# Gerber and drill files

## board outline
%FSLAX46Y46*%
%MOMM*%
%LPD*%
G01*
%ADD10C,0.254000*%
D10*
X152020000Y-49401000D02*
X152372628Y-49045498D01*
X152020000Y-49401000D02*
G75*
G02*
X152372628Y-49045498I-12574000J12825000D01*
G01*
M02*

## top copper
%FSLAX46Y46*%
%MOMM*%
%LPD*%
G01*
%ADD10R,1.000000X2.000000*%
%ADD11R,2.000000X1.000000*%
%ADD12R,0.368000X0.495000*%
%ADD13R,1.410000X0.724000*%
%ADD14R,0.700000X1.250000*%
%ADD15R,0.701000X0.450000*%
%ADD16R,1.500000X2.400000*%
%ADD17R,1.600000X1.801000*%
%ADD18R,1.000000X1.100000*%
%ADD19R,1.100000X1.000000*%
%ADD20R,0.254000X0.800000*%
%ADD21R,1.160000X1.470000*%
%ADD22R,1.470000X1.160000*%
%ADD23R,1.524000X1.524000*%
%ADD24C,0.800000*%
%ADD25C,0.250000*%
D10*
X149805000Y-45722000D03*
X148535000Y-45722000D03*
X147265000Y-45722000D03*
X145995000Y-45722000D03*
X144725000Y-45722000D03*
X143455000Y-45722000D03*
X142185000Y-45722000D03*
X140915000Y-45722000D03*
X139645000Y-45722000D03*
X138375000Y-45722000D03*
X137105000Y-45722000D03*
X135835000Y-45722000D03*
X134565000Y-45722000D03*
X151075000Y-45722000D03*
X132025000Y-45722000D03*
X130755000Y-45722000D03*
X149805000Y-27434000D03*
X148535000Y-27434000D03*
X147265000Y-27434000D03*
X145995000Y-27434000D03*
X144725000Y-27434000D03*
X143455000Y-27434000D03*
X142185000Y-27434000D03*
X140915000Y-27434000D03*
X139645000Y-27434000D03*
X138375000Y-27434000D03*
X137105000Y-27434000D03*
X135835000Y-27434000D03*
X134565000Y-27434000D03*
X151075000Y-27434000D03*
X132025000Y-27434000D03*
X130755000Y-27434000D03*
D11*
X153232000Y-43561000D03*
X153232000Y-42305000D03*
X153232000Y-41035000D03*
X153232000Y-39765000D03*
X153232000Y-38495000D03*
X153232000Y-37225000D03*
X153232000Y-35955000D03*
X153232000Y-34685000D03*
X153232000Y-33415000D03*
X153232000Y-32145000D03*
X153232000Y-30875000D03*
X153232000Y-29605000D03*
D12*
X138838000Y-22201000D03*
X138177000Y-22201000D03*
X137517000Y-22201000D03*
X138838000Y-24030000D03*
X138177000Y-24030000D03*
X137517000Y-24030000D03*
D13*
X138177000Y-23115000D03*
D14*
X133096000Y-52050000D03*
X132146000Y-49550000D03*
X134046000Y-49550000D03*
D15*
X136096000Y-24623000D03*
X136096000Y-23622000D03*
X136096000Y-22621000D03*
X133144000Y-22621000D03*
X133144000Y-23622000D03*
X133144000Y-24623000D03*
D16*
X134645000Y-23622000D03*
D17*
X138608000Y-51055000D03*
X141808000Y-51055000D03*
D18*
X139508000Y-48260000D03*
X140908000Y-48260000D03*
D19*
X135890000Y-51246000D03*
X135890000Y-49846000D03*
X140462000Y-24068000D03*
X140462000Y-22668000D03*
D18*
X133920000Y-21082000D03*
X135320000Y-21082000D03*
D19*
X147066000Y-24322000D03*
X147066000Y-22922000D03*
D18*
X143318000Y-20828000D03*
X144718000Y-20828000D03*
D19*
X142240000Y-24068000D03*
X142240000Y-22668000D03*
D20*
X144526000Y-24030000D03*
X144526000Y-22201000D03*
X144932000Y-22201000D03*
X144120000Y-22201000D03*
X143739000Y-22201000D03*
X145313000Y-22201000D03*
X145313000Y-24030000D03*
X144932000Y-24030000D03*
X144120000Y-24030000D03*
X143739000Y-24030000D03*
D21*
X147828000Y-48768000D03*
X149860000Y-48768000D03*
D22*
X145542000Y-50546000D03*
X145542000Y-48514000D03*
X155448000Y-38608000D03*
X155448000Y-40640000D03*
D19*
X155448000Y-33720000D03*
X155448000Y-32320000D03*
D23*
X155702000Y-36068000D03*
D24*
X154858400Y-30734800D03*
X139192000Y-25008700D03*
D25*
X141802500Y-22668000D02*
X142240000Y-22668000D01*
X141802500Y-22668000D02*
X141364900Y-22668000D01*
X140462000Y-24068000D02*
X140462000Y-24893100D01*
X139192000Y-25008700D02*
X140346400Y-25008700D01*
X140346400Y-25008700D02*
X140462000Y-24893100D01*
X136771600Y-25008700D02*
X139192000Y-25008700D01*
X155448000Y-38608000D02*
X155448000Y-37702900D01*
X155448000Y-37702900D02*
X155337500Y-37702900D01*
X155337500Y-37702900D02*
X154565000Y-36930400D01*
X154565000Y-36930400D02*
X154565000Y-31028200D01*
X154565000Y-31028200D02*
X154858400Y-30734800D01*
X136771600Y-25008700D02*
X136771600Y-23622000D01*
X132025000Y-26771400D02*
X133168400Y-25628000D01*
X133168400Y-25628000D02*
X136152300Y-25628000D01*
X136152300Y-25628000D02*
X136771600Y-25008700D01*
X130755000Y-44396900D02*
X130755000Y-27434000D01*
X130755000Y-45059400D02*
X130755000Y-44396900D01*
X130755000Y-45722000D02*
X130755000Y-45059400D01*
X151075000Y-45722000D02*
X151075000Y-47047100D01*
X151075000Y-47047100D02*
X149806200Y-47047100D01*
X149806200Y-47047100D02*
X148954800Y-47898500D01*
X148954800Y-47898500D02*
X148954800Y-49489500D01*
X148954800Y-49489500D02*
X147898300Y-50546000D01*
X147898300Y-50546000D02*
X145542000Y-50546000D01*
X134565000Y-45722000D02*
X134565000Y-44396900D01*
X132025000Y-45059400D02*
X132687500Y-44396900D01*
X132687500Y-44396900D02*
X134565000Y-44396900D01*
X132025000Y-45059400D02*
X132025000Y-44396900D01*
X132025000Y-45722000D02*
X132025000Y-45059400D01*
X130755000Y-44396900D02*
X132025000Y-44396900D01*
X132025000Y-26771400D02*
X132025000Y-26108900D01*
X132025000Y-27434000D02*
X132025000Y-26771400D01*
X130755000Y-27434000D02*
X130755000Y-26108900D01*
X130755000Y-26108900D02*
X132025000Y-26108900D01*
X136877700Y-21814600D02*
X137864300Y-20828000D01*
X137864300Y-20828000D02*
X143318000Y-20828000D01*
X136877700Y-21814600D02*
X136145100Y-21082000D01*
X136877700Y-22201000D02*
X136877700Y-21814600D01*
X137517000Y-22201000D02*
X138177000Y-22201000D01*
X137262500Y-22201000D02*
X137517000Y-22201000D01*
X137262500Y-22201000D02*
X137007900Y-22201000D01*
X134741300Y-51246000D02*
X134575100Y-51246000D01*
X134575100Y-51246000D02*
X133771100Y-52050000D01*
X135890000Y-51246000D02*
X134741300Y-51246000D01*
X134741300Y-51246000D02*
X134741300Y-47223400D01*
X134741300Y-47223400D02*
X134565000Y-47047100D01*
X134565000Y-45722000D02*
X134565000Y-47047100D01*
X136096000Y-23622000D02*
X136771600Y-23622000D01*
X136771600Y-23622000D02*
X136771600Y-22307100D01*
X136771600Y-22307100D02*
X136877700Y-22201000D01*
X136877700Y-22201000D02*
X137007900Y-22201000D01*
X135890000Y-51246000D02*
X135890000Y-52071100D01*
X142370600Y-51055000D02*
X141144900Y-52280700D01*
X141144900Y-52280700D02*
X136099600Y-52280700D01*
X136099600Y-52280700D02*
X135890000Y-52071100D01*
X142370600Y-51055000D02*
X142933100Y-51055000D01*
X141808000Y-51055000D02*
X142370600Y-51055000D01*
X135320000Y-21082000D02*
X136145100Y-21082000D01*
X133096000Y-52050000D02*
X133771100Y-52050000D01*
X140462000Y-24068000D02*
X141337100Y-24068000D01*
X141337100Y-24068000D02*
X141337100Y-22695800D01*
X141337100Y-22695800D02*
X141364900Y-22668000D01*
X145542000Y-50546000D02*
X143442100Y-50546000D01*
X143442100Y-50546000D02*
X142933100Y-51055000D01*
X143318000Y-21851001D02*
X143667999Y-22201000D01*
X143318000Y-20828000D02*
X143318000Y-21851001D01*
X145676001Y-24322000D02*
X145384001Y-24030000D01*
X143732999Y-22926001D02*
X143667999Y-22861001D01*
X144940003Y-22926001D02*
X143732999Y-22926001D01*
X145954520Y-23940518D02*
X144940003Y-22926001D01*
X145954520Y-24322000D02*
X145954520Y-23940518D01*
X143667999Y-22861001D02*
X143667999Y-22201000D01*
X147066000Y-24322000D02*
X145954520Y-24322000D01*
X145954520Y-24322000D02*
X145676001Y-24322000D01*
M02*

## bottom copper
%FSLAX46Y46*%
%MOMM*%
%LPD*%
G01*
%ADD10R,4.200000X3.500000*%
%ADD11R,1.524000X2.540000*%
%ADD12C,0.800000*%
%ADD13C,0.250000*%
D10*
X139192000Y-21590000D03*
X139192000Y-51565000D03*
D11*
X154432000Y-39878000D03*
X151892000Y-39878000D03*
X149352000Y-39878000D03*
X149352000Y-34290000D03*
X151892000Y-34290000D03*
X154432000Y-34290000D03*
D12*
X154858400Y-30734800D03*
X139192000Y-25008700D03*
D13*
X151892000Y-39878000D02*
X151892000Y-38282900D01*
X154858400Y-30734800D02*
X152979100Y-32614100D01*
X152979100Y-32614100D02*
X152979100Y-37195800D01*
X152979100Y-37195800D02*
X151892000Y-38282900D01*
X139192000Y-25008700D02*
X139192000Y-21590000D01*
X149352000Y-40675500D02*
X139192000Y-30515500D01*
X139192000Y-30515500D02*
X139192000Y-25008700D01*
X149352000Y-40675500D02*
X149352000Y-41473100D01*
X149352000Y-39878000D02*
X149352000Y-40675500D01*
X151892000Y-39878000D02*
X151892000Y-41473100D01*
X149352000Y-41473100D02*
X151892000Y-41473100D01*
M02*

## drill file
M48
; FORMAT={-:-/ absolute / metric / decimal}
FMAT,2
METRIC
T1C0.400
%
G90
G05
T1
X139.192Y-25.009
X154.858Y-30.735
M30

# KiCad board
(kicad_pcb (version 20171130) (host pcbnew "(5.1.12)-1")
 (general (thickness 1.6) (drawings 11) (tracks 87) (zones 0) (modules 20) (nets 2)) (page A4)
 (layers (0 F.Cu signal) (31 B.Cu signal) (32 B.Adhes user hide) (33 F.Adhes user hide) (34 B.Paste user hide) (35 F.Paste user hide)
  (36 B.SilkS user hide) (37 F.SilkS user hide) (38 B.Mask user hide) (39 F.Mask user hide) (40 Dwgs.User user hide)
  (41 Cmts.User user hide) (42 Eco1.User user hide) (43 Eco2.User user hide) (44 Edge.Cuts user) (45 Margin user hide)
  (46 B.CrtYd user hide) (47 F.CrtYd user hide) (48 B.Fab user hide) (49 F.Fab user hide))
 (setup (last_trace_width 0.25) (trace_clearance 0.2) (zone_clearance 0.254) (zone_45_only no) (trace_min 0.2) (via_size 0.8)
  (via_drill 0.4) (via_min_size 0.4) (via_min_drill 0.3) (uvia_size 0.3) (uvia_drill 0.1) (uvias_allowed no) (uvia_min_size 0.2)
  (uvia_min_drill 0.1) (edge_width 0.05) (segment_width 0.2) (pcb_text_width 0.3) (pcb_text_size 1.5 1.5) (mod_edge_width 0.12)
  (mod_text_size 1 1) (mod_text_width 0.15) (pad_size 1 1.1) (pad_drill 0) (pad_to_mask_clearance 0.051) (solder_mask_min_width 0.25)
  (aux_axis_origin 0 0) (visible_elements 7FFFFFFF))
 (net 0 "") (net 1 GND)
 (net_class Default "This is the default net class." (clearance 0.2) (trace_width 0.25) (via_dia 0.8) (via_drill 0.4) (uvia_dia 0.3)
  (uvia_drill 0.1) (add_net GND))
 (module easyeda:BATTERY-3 (layer F.Cu) (at 139.192 36.577)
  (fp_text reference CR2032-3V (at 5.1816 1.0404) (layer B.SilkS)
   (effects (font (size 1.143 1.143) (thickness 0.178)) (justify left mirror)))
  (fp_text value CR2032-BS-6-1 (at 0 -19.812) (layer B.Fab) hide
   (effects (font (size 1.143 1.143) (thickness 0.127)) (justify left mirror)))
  (pad 2 smd rect (at 0 -14.987 270) (size 3.5 4.2) (layers B.Cu B.Paste B.Mask) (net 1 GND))
  (pad 1 smd rect (at 0 14.988 270) (size 3.5 4.2) (layers B.Cu B.Paste B.Mask)))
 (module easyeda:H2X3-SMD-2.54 (layer F.Cu) (at 151.892 37.084 270)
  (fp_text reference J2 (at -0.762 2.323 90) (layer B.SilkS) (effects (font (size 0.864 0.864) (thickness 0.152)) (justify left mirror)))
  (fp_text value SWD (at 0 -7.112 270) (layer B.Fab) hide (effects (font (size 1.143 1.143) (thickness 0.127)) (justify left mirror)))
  (pad 1 smd rect (at 2.794 -2.54 270) (size 2.54 1.524) (layers B.Cu B.Paste B.Mask))
  (pad 2 smd rect (at 2.794 0 270) (size 2.54 1.524) (layers B.Cu B.Paste B.Mask) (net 1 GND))
  (pad 3 smd rect (at 2.794 2.54 270) (size 2.54 1.524) (layers B.Cu B.Paste B.Mask) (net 1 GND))
  (pad 4 smd rect (at -2.794 2.54 90) (size 2.54 1.524) (layers B.Cu B.Paste B.Mask))
  (pad 5 smd rect (at -2.794 0 90) (size 2.54 1.524) (layers B.Cu B.Paste B.Mask))
  (pad 6 smd rect (at -2.794 -2.54 90) (size 2.54 1.524) (layers B.Cu B.Paste B.Mask)))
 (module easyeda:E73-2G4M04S (layer F.Cu) (at 129.358 45.34 90)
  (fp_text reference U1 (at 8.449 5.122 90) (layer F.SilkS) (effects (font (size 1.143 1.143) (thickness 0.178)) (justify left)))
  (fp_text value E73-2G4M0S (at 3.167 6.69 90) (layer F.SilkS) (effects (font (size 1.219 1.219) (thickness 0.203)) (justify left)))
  (pad 14 smd rect (at -0.382 20.447 90) (size 2 1) (layers F.Cu F.Paste F.Mask))
  (pad 13 smd rect (at -0.382 19.177 90) (size 2 1) (layers F.Cu F.Paste F.Mask))
  (pad 12 smd rect (at -0.382 17.907 90) (size 2 1) (layers F.Cu F.Paste F.Mask))
  (pad 11 smd rect (at -0.382 16.637 90) (size 2 1) (layers F.Cu F.Paste F.Mask))
  (pad 10 smd rect (at -0.382 15.367 90) (size 2 1) (layers F.Cu F.Paste F.Mask))
  (pad 9 smd rect (at -0.382 14.097 90) (size 2 1) (layers F.Cu F.Paste F.Mask))
  (pad 8 smd rect (at -0.382 12.827 90) (size 2 1) (layers F.Cu F.Paste F.Mask))
  (pad 7 smd rect (at -0.382 11.557 90) (size 2 1) (layers F.Cu F.Paste F.Mask))
  (pad 6 smd rect (at -0.382 10.287 90) (size 2 1) (layers F.Cu F.Paste F.Mask))
  (pad 5 smd rect (at -0.382 9.017 90) (size 2 1) (layers F.Cu F.Paste F.Mask))
  (pad 4 smd rect (at -0.382 7.747 90) (size 2 1) (layers F.Cu F.Paste F.Mask))
  (pad 3 smd rect (at -0.382 6.477 90) (size 2 1) (layers F.Cu F.Paste F.Mask))
  (pad 2 smd rect (at -0.382 5.207 90) (size 2 1) (layers F.Cu F.Paste F.Mask) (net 1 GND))
  (pad 15 smd rect (at -0.382 21.717 90) (size 2 1) (layers F.Cu F.Paste F.Mask) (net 1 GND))
  (pad 1 smd rect (at -0.382 2.667 90) (size 2 1) (layers F.Cu F.Paste F.Mask) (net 1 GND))
  (pad 0 smd rect (at -0.382 1.397 90) (size 2 1) (layers F.Cu F.Paste F.Mask) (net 1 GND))
  (pad 29 smd rect (at 17.906 20.447 90) (size 2 1) (layers F.Cu F.Paste F.Mask))
  (pad 30 smd rect (at 17.906 19.177 90) (size 2 1) (layers F.Cu F.Paste F.Mask))
  (pad 31 smd rect (at 17.906 17.907 90) (size 2 1) (layers F.Cu F.Paste F.Mask))
  (pad 32 smd rect (at 17.906 16.637 90) (size 2 1) (layers F.Cu F.Paste F.Mask))
  (pad 33 smd rect (at 17.906 15.367 90) (size 2 1) (layers F.Cu F.Paste F.Mask))
  (pad 34 smd rect (at 17.906 14.097 90) (size 2 1) (layers F.Cu F.Paste F.Mask))
  (pad 35 smd rect (at 17.906 12.827 90) (size 2 1) (layers F.Cu F.Paste F.Mask))
  (pad 36 smd rect (at 17.906 11.557 90) (size 2 1) (layers F.Cu F.Paste F.Mask))
  (pad 37 smd rect (at 17.906 10.287 90) (size 2 1) (layers F.Cu F.Paste F.Mask))
  (pad 38 smd rect (at 17.906 9.017 90) (size 2 1) (layers F.Cu F.Paste F.Mask))
  (pad 39 smd rect (at 17.906 7.747 90) (size 2 1) (layers F.Cu F.Paste F.Mask))
  (pad 40 smd rect (at 17.906 6.477 90) (size 2 1) (layers F.Cu F.Paste F.Mask))
  (pad 41 smd rect (at 17.906 5.207 90) (size 2 1) (layers F.Cu F.Paste F.Mask))
  (pad 28 smd rect (at 17.906 21.717 90) (size 2 1) (layers F.Cu F.Paste F.Mask))
  (pad 42 smd rect (at 17.906 2.667 90) (size 2 1) (layers F.Cu F.Paste F.Mask) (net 1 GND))
  (pad 43 smd rect (at 17.906 1.397 90) (size 2 1) (layers F.Cu F.Paste F.Mask) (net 1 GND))
  (pad 16 smd rect (at 1.779 23.874 180) (size 2 1) (layers F.Cu F.Paste F.Mask))
  (pad 17 smd rect (at 3.035 23.874 180) (size 2 1) (layers F.Cu F.Paste F.Mask))
  (pad 18 smd rect (at 4.305 23.874 180) (size 2 1) (layers F.Cu F.Paste F.Mask))
  (pad 19 smd rect (at 5.575 23.874 180) (size 2 1) (layers F.Cu F.Paste F.Mask))
  (pad 20 smd rect (at 6.845 23.874 180) (size 2 1) (layers F.Cu F.Paste F.Mask))
  (pad 21 smd rect (at 8.115 23.874 180) (size 2 1) (layers F.Cu F.Paste F.Mask))
  (pad 22 smd rect (at 9.385 23.874 180) (size 2 1) (layers F.Cu F.Paste F.Mask))
  (pad 23 smd rect (at 10.655 23.874 180) (size 2 1) (layers F.Cu F.Paste F.Mask))
  (pad 24 smd rect (at 11.925 23.874 180) (size 2 1) (layers F.Cu F.Paste F.Mask))
  (pad 25 smd rect (at 13.195 23.874 180) (size 2 1) (layers F.Cu F.Paste F.Mask))
  (pad 26 smd rect (at 14.465 23.874 180) (size 2 1) (layers F.Cu F.Paste F.Mask))
  (pad 27 smd rect (at 15.735 23.874 180) (size 2 1) (layers F.Cu F.Paste F.Mask)))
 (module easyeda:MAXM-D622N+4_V (layer F.Cu) (at 138.176 23.114 270)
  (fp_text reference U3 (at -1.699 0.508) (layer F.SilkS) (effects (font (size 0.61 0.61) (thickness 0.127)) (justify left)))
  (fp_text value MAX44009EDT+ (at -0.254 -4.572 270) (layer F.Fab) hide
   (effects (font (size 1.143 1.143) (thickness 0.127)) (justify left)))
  (pad 1 smd rect (at -0.913 -0.662) (size 0.368 0.495) (layers F.Cu F.Paste F.Mask))
  (pad 2 smd rect (at -0.913 -0.001) (size 0.368 0.495) (layers F.Cu F.Paste F.Mask) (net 1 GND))
  (pad 3 smd rect (at -0.913 0.659) (size 0.368 0.495) (layers F.Cu F.Paste F.Mask) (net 1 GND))
  (pad 6 smd rect (at 0.916 -0.662) (size 0.368 0.495) (layers F.Cu F.Paste F.Mask))
  (pad 5 smd rect (at 0.916 -0.001) (size 0.368 0.495) (layers F.Cu F.Paste F.Mask))
  (pad 4 smd rect (at 0.916 0.659) (size 0.368 0.495) (layers F.Cu F.Paste F.Mask))
  (pad 7 smd rect (at 0.001 -0.001) (size 1.41 0.724) (layers F.Cu F.Paste F.Mask)))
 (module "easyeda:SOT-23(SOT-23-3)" (layer F.Cu) (at 133.096 50.8 180)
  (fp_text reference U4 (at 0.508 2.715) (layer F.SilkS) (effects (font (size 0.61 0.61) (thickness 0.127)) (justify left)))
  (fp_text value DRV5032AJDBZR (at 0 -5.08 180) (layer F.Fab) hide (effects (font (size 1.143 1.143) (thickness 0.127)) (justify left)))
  (pad 3 smd rect (at 0 -1.25) (size 0.7 1.25) (layers F.Cu F.Paste F.Mask) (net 1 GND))
  (pad 2 smd rect (at 0.95 1.25) (size 0.7 1.25) (layers F.Cu F.Paste F.Mask))
  (pad 1 smd rect (at -0.95 1.25) (size 0.7 1.25) (layers F.Cu F.Paste F.Mask)))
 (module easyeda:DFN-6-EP (layer F.Cu) (at 134.62 23.622 90)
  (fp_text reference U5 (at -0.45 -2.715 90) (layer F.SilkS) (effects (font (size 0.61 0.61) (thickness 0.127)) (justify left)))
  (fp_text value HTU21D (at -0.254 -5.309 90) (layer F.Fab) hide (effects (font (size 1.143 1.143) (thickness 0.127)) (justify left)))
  (pad 1 smd rect (at -1.001 1.476 90) (size 0.45 0.701) (layers F.Cu F.Paste F.Mask))
  (pad 2 smd rect (at 0 1.476 90) (size 0.45 0.701) (layers F.Cu F.Paste F.Mask) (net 1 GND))
  (pad 3 smd rect (at 1.001 1.476 90) (size 0.45 0.701) (layers F.Cu F.Paste F.Mask))
  (pad 4 smd rect (at 1.001 -1.476 90) (size 0.45 0.701) (layers F.Cu F.Paste F.Mask))
  (pad 5 smd rect (at 0 -1.476 90) (size 0.45 0.701) (layers F.Cu F.Paste F.Mask))
  (pad 6 smd rect (at -1.001 -1.476 90) (size 0.45 0.701) (layers F.Cu F.Paste F.Mask))
  (pad 7 smd rect (at 0 0.025 90) (size 2.4 1.5) (layers F.Cu F.Paste F.Mask)))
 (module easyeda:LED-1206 (layer F.Cu) (at 140.208 51.054 180)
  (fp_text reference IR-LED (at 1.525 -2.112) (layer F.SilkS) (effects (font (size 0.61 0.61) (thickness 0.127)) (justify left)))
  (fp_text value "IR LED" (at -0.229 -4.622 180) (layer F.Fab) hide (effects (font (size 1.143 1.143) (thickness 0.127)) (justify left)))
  (pad 1 smd rect (at 1.6 -0.001) (size 1.6 1.801) (layers F.Cu F.Paste F.Mask))
  (pad 2 smd rect (at -1.6 -0.001) (size 1.6 1.801) (layers F.Cu F.Paste F.Mask) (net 1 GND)))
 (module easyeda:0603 (layer F.Cu) (at 140.208 48.26)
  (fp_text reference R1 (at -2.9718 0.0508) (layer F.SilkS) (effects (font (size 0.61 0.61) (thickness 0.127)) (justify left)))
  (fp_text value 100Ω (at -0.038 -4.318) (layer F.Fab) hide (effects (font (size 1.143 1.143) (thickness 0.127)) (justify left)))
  (pad 1 smd rect (at -0.7 0) (size 1 1.1) (layers F.Cu F.Paste F.Mask))
  (pad 2 smd rect (at 0.7 0) (size 1 1.1) (layers F.Cu F.Paste F.Mask)))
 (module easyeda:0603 (layer F.Cu) (at 135.89 50.546 90)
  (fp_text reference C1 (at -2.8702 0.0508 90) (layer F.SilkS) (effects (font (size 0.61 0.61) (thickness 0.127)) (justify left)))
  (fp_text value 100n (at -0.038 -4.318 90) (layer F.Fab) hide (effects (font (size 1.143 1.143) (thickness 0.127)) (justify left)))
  (pad 1 smd rect (at -0.7 0 90) (size 1 1.1) (layers F.Cu F.Paste F.Mask) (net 1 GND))
  (pad 2 smd rect (at 0.7 0 90) (size 1 1.1) (layers F.Cu F.Paste F.Mask)))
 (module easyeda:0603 (layer F.Cu) (at 140.462 23.368 90)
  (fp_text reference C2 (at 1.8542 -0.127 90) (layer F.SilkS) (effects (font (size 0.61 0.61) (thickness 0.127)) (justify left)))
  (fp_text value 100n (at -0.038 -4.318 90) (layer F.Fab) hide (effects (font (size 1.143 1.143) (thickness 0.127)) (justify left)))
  (pad 1 smd rect (at -0.7 0 90) (size 1 1.1) (layers F.Cu F.Paste F.Mask) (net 1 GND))
  (pad 2 smd rect (at 0.7 0 90) (size 1 1.1) (layers F.Cu F.Paste F.Mask)))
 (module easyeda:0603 (layer F.Cu) (at 134.62 21.082)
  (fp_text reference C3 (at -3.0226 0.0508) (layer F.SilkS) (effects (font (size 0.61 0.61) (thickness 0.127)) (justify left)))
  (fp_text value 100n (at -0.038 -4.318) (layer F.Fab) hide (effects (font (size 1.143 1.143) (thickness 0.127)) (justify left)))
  (pad 1 smd rect (at -0.7 0) (size 1 1.1) (layers F.Cu F.Paste F.Mask))
  (pad 2 smd rect (at 0.7 0) (size 1 1.1) (layers F.Cu F.Paste F.Mask) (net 1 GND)))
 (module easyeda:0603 (layer F.Cu) (at 147.066 23.622 90)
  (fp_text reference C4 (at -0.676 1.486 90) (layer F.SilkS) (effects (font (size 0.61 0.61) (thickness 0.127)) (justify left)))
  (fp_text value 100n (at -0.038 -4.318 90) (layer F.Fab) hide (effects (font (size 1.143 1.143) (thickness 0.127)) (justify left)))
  (pad 1 smd rect (at -0.7 0 90) (size 1 1.1) (layers F.Cu F.Paste F.Mask) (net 1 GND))
  (pad 2 smd rect (at 0.7 0 90) (size 1 1.1) (layers F.Cu F.Paste F.Mask)))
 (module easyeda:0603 (layer F.Cu) (at 144.018 20.828)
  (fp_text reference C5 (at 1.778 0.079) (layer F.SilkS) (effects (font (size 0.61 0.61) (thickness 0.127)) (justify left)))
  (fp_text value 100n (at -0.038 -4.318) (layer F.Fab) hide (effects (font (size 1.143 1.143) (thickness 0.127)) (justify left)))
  (pad 1 smd rect (at -0.7 0) (size 1 1.1) (layers F.Cu F.Paste F.Mask) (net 1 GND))
  (pad 2 smd rect (at 0.7 0) (size 1 1.1) (layers F.Cu F.Paste F.Mask)))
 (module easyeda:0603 (layer F.Cu) (at 142.24 23.368 90)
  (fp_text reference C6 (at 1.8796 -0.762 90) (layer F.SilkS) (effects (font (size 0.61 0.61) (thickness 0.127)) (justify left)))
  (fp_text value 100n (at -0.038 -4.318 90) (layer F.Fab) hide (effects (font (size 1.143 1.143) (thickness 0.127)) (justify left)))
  (pad 1 smd rect (at -0.7 0 90) (size 1 1.1) (layers F.Cu F.Paste F.Mask))
  (pad 2 smd rect (at 0.7 0 90) (size 1 1.1) (layers F.Cu F.Paste F.Mask) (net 1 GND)))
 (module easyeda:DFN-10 (layer F.Cu) (at 144.526 23.114 270)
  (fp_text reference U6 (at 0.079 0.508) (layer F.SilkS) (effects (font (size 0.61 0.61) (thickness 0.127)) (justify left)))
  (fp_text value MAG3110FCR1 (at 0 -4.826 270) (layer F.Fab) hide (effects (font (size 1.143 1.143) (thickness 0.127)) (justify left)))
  (pad 8 smd rect (at 0.916 0 270) (size 0.8 0.254) (layers F.Cu F.Paste F.Mask))
  (pad 3 smd rect (at -0.913 0 270) (size 0.8 0.254) (layers F.Cu F.Paste F.Mask))
  (pad 2 smd rect (at -0.913 -0.406 270) (size 0.8 0.254) (layers F.Cu F.Paste F.Mask))
  (pad 4 smd rect (at -0.913 0.406 270) (size 0.8 0.254) (layers F.Cu F.Paste F.Mask))
  (pad 5 smd rect (at -0.913 0.787 270) (size 0.8 0.254) (layers F.Cu F.Paste F.Mask) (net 1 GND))
  (pad 1 smd rect (at -0.913 -0.787 270) (size 0.8 0.254) (layers F.Cu F.Paste F.Mask))
  (pad 10 smd rect (at 0.916 -0.787 270) (size 0.8 0.254) (layers F.Cu F.Paste F.Mask) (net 1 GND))
  (pad 9 smd rect (at 0.916 -0.406 270) (size 0.8 0.254) (layers F.Cu F.Paste F.Mask))
  (pad 7 smd rect (at 0.916 0.406 270) (size 0.8 0.254) (layers F.Cu F.Paste F.Mask))
  (pad 6 smd rect (at 0.916 0.787 270) (size 0.8 0.254) (layers F.Cu F.Paste F.Mask)))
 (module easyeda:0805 (layer F.Cu) (at 147.828 48.768)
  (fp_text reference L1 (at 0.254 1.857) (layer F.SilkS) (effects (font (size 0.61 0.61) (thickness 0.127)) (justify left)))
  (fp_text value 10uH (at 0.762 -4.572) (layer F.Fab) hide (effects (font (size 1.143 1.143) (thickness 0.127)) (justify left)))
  (pad 1 smd rect (at 0 0) (size 1.16 1.47) (layers F.Cu F.Paste F.Mask))
  (pad 2 smd rect (at 2.032 0) (size 1.16 1.47) (layers F.Cu F.Paste F.Mask)))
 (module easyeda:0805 (layer F.Cu) (at 145.542 50.546 90)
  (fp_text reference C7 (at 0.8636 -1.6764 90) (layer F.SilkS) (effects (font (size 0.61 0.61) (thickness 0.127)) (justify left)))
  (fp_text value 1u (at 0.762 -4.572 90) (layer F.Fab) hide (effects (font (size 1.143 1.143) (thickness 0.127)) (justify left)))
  (pad 1 smd rect (at 0 0 90) (size 1.16 1.47) (layers F.Cu F.Paste F.Mask) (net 1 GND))
  (pad 2 smd rect (at 2.032 0 90) (size 1.16 1.47) (layers F.Cu F.Paste F.Mask)))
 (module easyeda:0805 (layer F.Cu) (at 155.448 38.608 270)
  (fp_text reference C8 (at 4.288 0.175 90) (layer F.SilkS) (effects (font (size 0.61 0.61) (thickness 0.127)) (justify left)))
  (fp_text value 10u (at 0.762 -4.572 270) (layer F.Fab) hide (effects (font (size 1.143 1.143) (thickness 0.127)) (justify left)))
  (pad 1 smd rect (at 0 0 270) (size 1.16 1.47) (layers F.Cu F.Paste F.Mask) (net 1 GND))
  (pad 2 smd rect (at 2.032 0 270) (size 1.16 1.47) (layers F.Cu F.Paste F.Mask)))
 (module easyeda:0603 (layer F.Cu) (at 155.448 33.02 90)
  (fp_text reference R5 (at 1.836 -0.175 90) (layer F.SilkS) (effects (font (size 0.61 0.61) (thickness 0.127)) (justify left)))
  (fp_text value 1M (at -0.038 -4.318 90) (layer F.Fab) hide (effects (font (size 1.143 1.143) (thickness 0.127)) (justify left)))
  (pad 1 smd rect (at -0.7 0 90) (size 1 1.1) (layers F.Cu F.Paste F.Mask))
  (pad 2 smd rect (at 0.7 0 90) (size 1 1.1) (layers F.Cu F.Paste F.Mask)))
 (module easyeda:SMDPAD (layer F.Cu) (at 155.702 36.068)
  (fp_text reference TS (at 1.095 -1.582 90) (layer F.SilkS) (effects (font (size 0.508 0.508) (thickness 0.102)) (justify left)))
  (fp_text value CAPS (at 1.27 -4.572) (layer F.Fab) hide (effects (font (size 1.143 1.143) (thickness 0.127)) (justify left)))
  (pad 1 smd rect (at 0 0) (size 1.524 1.524) (layers F.Cu F.Paste F.Mask)))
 (gr_line (start 152.02 49.401) (end 152.372628 49.045498) (layer Edge.Cuts) (width 0.254))
 (gr_arc (start 139.446 36.576) (end 152.02 49.401) (angle 358.4025929) (layer Edge.Cuts) (width 0.254))
 (segment (start 141.8025 22.668) (end 142.24 22.668) (width 0.25) (layer F.Cu) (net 1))
 (segment (start 141.8025 22.668) (end 141.3649 22.668) (width 0.25) (layer F.Cu) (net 1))
 (segment (start 140.462 24.068) (end 140.462 24.8931) (width 0.25) (layer F.Cu) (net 1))
 (segment (start 139.192 25.0087) (end 140.3464 25.0087) (width 0.25) (layer F.Cu) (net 1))
 (segment (start 140.3464 25.0087) (end 140.462 24.8931) (width 0.25) (layer F.Cu) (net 1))
 (segment (start 136.7716 25.0087) (end 139.192 25.0087) (width 0.25) (layer F.Cu) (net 1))
 (segment (start 155.448 38.608) (end 155.448 37.7029) (width 0.25) (layer F.Cu) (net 1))
 (segment (start 151.892 39.878) (end 151.892 38.2829) (width 0.25) (layer B.Cu) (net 1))
 (segment (start 155.448 37.7029) (end 155.3375 37.7029) (width 0.25) (layer F.Cu) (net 1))
 (segment (start 155.3375 37.7029) (end 154.565 36.9304) (width 0.25) (layer F.Cu) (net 1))
 (segment (start 154.565 36.9304) (end 154.565 31.0282) (width 0.25) (layer F.Cu) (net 1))
 (segment (start 154.565 31.0282) (end 154.8584 30.7348) (width 0.25) (layer F.Cu) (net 1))
 (segment (start 154.8584 30.7348) (end 152.9791 32.6141) (width 0.25) (layer B.Cu) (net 1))
 (segment (start 152.9791 32.6141) (end 152.9791 37.1958) (width 0.25) (layer B.Cu) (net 1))
 (segment (start 152.9791 37.1958) (end 151.892 38.2829) (width 0.25) (layer B.Cu) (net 1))
 (segment (start 139.192 25.0087) (end 139.192 21.59) (width 0.25) (layer B.Cu) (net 1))
 (segment (start 149.352 40.6755) (end 139.192 30.5155) (width 0.25) (layer B.Cu) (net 1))
 (segment (start 139.192 30.5155) (end 139.192 25.0087) (width 0.25) (layer B.Cu) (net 1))
 (segment (start 136.7716 25.0087) (end 136.7716 23.622) (width 0.25) (layer F.Cu) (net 1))
 (segment (start 132.025 26.7714) (end 133.1684 25.628) (width 0.25) (layer F.Cu) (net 1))
 (segment (start 133.1684 25.628) (end 136.1523 25.628) (width 0.25) (layer F.Cu) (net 1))
 (segment (start 136.1523 25.628) (end 136.7716 25.0087) (width 0.25) (layer F.Cu) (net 1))
 (segment (start 149.352 40.6755) (end 149.352 41.4731) (width 0.25) (layer B.Cu) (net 1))
 (segment (start 149.352 39.878) (end 149.352 40.6755) (width 0.25) (layer B.Cu) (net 1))
 (segment (start 151.892 39.878) (end 151.892 41.4731) (width 0.25) (layer B.Cu) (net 1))
 (segment (start 149.352 41.4731) (end 151.892 41.4731) (width 0.25) (layer B.Cu) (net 1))
 (segment (start 130.755 44.3969) (end 130.755 27.434) (width 0.25) (layer F.Cu) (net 1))
 (segment (start 130.755 45.0594) (end 130.755 44.3969) (width 0.25) (layer F.Cu) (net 1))
 (segment (start 130.755 45.722) (end 130.755 45.0594) (width 0.25) (layer F.Cu) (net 1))
 (segment (start 151.075 45.722) (end 151.075 47.0471) (width 0.25) (layer F.Cu) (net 1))
 (segment (start 151.075 47.0471) (end 149.8062 47.0471) (width 0.25) (layer F.Cu) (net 1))
 (segment (start 149.8062 47.0471) (end 148.9548 47.8985) (width 0.25) (layer F.Cu) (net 1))
 (segment (start 148.9548 47.8985) (end 148.9548 49.4895) (width 0.25) (layer F.Cu) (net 1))
 (segment (start 148.9548 49.4895) (end 147.8983 50.546) (width 0.25) (layer F.Cu) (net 1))
 (segment (start 147.8983 50.546) (end 145.542 50.546) (width 0.25) (layer F.Cu) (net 1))
 (segment (start 134.565 45.722) (end 134.565 44.3969) (width 0.25) (layer F.Cu) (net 1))
 (segment (start 132.025 45.0594) (end 132.6875 44.3969) (width 0.25) (layer F.Cu) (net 1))
 (segment (start 132.6875 44.3969) (end 134.565 44.3969) (width 0.25) (layer F.Cu) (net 1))
 (segment (start 132.025 45.0594) (end 132.025 44.3969) (width 0.25) (layer F.Cu) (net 1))
 (segment (start 132.025 45.722) (end 132.025 45.0594) (width 0.25) (layer F.Cu) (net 1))
 (segment (start 130.755 44.3969) (end 132.025 44.3969) (width 0.25) (layer F.Cu) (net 1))
 (segment (start 132.025 26.7714) (end 132.025 26.1089) (width 0.25) (layer F.Cu) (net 1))
 (segment (start 132.025 27.434) (end 132.025 26.7714) (width 0.25) (layer F.Cu) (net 1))
 (segment (start 130.755 27.434) (end 130.755 26.1089) (width 0.25) (layer F.Cu) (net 1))
 (segment (start 130.755 26.1089) (end 132.025 26.1089) (width 0.25) (layer F.Cu) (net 1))
 (segment (start 136.8777 21.8146) (end 137.8643 20.828) (width 0.25) (layer F.Cu) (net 1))
 (segment (start 137.8643 20.828) (end 143.318 20.828) (width 0.25) (layer F.Cu) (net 1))
 (segment (start 136.8777 21.8146) (end 136.1451 21.082) (width 0.25) (layer F.Cu) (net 1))
 (segment (start 136.8777 22.201) (end 136.8777 21.8146) (width 0.25) (layer F.Cu) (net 1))
 (segment (start 137.517 22.201) (end 138.177 22.201) (width 0.25) (layer F.Cu) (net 1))
 (segment (start 137.2625 22.201) (end 137.517 22.201) (width 0.25) (layer F.Cu) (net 1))
 (segment (start 137.2625 22.201) (end 137.0079 22.201) (width 0.25) (layer F.Cu) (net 1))
 (segment (start 134.7413 51.246) (end 134.5751 51.246) (width 0.25) (layer F.Cu) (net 1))
 (segment (start 134.5751 51.246) (end 133.7711 52.05) (width 0.25) (layer F.Cu) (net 1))
 (segment (start 135.89 51.246) (end 134.7413 51.246) (width 0.25) (layer F.Cu) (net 1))
 (segment (start 134.7413 51.246) (end 134.7413 47.2234) (width 0.25) (layer F.Cu) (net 1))
 (segment (start 134.7413 47.2234) (end 134.565 47.0471) (width 0.25) (layer F.Cu) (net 1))
 (segment (start 134.565 45.722) (end 134.565 47.0471) (width 0.25) (layer F.Cu) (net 1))
 (segment (start 136.096 23.622) (end 136.7716 23.622) (width 0.25) (layer F.Cu) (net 1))
 (segment (start 136.7716 23.622) (end 136.7716 22.3071) (width 0.25) (layer F.Cu) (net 1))
 (segment (start 136.7716 22.3071) (end 136.8777 22.201) (width 0.25) (layer F.Cu) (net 1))
 (segment (start 136.8777 22.201) (end 137.0079 22.201) (width 0.25) (layer F.Cu) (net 1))
 (segment (start 135.89 51.246) (end 135.89 52.0711) (width 0.25) (layer F.Cu) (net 1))
 (segment (start 142.3706 51.055) (end 141.1449 52.2807) (width 0.25) (layer F.Cu) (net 1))
 (segment (start 141.1449 52.2807) (end 136.0996 52.2807) (width 0.25) (layer F.Cu) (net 1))
 (segment (start 136.0996 52.2807) (end 135.89 52.0711) (width 0.25) (layer F.Cu) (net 1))
 (segment (start 142.3706 51.055) (end 142.9331 51.055) (width 0.25) (layer F.Cu) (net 1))
 (segment (start 141.808 51.055) (end 142.3706 51.055) (width 0.25) (layer F.Cu) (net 1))
 (segment (start 135.32 21.082) (end 136.1451 21.082) (width 0.25) (layer F.Cu) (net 1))
 (segment (start 133.096 52.05) (end 133.7711 52.05) (width 0.25) (layer F.Cu) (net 1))
 (segment (start 140.462 24.068) (end 141.3371 24.068) (width 0.25) (layer F.Cu) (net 1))
 (segment (start 141.3371 24.068) (end 141.3371 22.6958) (width 0.25) (layer F.Cu) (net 1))
 (segment (start 141.3371 22.6958) (end 141.3649 22.668) (width 0.25) (layer F.Cu) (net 1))
 (segment (start 145.542 50.546) (end 143.4421 50.546) (width 0.25) (layer F.Cu) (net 1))
 (segment (start 143.4421 50.546) (end 142.9331 51.055) (width 0.25) (layer F.Cu) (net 1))
 (via (at 154.8584 30.7348) (size 0.8) (layers F.Cu B.Cu) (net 1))
 (via (at 139.192 25.0087) (size 0.8) (layers F.Cu B.Cu) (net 1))
 (segment (start 143.318 21.851001) (end 143.667999 22.201) (width 0.25) (layer F.Cu) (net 1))
 (segment (start 143.318 20.828) (end 143.318 21.851001) (width 0.25) (layer F.Cu) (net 1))
 (segment (start 145.676001 24.322) (end 145.384001 24.03) (width 0.25) (layer F.Cu) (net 1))
 (segment (start 143.732999 22.926001) (end 143.667999 22.861001) (width 0.25) (layer F.Cu) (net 1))
 (segment (start 144.940003 22.926001) (end 143.732999 22.926001) (width 0.25) (layer F.Cu) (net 1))
 (segment (start 145.95452 23.940518) (end 144.940003 22.926001) (width 0.25) (layer F.Cu) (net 1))
 (segment (start 145.95452 24.322) (end 145.95452 23.940518) (width 0.25) (layer F.Cu) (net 1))
 (segment (start 143.667999 22.861001) (end 143.667999 22.201) (width 0.25) (layer F.Cu) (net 1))
 (segment (start 147.066 24.322) (end 145.95452 24.322) (width 0.25) (layer F.Cu) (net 1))
 (segment (start 145.95452 24.322) (end 145.676001 24.322) (width 0.25) (layer F.Cu) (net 1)))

